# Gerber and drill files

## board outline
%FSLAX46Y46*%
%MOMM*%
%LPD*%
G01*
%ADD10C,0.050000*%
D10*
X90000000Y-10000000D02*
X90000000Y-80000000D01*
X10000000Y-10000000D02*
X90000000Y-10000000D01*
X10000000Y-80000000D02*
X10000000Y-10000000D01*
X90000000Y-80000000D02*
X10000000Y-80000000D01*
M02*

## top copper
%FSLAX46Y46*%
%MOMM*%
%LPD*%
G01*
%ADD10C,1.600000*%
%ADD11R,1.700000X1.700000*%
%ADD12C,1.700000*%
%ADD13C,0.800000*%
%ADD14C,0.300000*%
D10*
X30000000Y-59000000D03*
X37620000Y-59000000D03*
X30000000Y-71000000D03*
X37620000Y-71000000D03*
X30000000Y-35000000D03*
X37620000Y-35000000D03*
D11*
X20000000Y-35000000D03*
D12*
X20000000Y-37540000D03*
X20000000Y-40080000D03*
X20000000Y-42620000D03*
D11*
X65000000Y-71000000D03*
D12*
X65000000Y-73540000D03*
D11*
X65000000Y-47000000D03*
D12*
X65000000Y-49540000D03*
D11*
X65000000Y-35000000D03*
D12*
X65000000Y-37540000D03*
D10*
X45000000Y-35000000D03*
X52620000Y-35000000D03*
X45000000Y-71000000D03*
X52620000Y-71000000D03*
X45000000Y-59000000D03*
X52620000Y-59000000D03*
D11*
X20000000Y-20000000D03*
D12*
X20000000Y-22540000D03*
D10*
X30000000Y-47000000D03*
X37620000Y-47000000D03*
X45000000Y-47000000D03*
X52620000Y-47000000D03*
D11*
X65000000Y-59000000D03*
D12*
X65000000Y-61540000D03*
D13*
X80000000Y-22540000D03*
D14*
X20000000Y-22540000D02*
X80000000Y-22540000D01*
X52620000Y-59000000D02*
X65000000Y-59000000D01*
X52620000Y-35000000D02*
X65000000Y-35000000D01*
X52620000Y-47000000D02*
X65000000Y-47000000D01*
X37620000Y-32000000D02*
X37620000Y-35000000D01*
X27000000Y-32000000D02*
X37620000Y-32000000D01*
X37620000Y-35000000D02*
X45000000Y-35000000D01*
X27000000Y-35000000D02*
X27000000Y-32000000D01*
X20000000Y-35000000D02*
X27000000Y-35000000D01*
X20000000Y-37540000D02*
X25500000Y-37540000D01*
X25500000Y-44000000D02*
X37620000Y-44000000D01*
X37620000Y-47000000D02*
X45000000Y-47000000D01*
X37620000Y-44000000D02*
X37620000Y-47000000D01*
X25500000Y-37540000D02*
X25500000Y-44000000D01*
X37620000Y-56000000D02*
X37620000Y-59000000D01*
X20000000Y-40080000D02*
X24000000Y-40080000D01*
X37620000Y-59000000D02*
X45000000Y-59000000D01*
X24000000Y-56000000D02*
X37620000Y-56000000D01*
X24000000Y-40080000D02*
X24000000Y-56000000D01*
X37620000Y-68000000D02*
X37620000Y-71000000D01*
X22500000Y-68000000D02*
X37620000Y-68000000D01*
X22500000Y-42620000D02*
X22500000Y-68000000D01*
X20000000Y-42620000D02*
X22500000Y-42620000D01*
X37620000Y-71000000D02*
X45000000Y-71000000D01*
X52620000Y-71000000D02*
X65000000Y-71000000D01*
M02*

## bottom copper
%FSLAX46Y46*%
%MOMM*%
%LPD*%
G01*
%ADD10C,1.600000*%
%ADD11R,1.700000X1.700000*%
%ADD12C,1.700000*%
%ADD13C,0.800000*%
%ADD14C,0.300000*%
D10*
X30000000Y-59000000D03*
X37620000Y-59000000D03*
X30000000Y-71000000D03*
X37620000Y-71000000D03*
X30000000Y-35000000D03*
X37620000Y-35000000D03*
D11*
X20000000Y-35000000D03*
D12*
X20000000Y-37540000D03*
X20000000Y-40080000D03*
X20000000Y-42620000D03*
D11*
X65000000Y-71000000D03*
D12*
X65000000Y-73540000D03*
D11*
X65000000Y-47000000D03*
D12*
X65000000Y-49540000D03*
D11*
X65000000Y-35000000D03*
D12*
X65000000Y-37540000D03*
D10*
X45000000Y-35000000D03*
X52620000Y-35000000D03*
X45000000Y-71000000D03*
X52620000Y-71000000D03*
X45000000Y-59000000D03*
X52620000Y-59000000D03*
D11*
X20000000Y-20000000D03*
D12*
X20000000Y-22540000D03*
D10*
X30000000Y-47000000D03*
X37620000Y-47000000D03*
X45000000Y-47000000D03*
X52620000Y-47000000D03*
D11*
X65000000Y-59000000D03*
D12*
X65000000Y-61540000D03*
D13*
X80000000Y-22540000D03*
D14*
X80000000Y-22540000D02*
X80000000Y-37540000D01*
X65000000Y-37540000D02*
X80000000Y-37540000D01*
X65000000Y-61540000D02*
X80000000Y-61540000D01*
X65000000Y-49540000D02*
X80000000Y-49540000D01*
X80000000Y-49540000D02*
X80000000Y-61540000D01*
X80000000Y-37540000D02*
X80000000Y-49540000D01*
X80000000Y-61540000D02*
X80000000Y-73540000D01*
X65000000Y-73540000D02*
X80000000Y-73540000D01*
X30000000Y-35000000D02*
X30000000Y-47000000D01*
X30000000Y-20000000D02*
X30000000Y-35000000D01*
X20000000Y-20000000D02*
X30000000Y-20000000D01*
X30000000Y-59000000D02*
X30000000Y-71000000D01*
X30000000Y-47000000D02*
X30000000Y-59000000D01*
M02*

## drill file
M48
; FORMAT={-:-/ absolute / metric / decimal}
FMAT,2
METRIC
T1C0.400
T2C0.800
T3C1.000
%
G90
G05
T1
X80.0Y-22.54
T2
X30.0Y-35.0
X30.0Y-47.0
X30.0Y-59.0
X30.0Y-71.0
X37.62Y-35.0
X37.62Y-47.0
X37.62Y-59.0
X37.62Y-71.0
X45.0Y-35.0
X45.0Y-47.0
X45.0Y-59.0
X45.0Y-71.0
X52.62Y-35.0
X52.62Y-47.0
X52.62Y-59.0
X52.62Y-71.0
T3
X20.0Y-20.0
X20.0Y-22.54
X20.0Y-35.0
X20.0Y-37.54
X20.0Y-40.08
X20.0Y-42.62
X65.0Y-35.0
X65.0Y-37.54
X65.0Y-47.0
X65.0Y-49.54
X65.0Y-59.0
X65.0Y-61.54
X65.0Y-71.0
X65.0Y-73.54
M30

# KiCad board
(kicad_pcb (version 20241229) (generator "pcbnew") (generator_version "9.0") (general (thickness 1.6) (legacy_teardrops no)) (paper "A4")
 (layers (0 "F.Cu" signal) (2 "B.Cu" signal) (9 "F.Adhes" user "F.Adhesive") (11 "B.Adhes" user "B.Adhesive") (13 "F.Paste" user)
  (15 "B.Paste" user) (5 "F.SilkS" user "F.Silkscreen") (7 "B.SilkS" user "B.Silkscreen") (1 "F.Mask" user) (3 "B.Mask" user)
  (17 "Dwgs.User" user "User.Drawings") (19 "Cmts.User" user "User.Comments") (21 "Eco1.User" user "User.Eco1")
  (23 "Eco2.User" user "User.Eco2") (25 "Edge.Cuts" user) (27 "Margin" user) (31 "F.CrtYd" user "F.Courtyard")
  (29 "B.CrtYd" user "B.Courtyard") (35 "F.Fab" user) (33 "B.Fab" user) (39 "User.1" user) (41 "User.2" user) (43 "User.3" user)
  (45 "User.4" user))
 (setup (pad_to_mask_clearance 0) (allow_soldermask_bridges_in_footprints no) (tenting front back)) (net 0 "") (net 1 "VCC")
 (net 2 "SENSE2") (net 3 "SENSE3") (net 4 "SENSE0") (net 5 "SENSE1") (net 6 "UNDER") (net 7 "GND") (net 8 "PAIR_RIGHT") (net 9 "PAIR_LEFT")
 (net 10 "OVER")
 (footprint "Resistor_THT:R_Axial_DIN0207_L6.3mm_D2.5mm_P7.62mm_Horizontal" (layer "F.Cu") (at 30 59)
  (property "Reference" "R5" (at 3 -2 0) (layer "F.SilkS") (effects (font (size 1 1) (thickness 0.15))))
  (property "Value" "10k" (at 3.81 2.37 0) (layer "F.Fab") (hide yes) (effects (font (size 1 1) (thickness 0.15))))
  (pad "1" thru_hole circle (at 0 0) (size 1.6 1.6) (drill 0.8) (layers "*.Cu" "*.Mask") (remove_unused_layers no) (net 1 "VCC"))
  (pad "2" thru_hole circle (at 7.62 0) (size 1.6 1.6) (drill 0.8) (layers "*.Cu" "*.Mask") (remove_unused_layers no) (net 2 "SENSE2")))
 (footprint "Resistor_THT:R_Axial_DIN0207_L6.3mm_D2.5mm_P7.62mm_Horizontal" (layer "F.Cu") (at 30 71)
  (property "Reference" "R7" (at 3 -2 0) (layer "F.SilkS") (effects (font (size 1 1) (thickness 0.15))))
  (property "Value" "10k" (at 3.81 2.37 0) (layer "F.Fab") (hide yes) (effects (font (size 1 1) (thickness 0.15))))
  (pad "1" thru_hole circle (at 0 0) (size 1.6 1.6) (drill 0.8) (layers "*.Cu" "*.Mask") (remove_unused_layers no) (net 1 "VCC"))
  (pad "2" thru_hole circle (at 7.62 0) (size 1.6 1.6) (drill 0.8) (layers "*.Cu" "*.Mask") (remove_unused_layers no) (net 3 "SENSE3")))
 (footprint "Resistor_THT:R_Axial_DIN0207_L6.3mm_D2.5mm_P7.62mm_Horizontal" (layer "F.Cu") (at 30 35)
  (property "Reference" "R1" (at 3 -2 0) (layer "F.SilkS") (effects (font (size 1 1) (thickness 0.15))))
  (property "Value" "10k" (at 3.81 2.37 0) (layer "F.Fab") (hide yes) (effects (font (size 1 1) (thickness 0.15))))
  (pad "1" thru_hole circle (at 0 0) (size 1.6 1.6) (drill 0.8) (layers "*.Cu" "*.Mask") (remove_unused_layers no) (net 1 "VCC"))
  (pad "2" thru_hole circle (at 7.62 0) (size 1.6 1.6) (drill 0.8) (layers "*.Cu" "*.Mask") (remove_unused_layers no) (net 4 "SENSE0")))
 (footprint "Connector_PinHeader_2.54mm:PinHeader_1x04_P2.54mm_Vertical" (layer "F.Cu") (at 20 35)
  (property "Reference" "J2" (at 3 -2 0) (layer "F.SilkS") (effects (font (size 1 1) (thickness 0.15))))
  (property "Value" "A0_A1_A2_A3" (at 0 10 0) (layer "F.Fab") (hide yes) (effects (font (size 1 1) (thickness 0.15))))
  (pad "1" thru_hole rect (at 0 0) (size 1.7 1.7) (drill 1) (layers "*.Cu" "*.Mask") (remove_unused_layers no) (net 4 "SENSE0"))
  (pad "2" thru_hole circle (at 0 2.54) (size 1.7 1.7) (drill 1) (layers "*.Cu" "*.Mask") (remove_unused_layers no) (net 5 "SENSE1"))
  (pad "3" thru_hole circle (at 0 5.08) (size 1.7 1.7) (drill 1) (layers "*.Cu" "*.Mask") (remove_unused_layers no) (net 2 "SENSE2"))
  (pad "4" thru_hole circle (at 0 7.62) (size 1.7 1.7) (drill 1) (layers "*.Cu" "*.Mask") (remove_unused_layers no) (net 3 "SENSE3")))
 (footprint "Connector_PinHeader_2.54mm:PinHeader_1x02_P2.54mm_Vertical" (layer "F.Cu") (at 65 71)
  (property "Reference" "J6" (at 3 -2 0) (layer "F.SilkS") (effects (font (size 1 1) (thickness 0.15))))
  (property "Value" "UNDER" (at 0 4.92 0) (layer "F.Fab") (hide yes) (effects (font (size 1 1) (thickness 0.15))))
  (pad "1" thru_hole rect (at 0 0) (size 1.7 1.7) (drill 1) (layers "*.Cu" "*.Mask") (remove_unused_layers no) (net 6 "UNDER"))
  (pad "2" thru_hole circle (at 0 2.54) (size 1.7 1.7) (drill 1) (layers "*.Cu" "*.Mask") (remove_unused_layers no) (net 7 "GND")))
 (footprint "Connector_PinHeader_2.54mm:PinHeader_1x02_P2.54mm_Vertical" (layer "F.Cu") (at 65 47)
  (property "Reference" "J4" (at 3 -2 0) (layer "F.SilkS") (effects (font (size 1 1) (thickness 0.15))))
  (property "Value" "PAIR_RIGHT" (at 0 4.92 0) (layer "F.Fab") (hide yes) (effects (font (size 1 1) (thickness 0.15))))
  (pad "1" thru_hole rect (at 0 0) (size 1.7 1.7) (drill 1) (layers "*.Cu" "*.Mask") (remove_unused_layers no) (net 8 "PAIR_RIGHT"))
  (pad "2" thru_hole circle (at 0 2.54) (size 1.7 1.7) (drill 1) (layers "*.Cu" "*.Mask") (remove_unused_layers no) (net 7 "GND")))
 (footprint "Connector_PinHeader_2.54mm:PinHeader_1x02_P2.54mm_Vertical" (layer "F.Cu") (at 65 35)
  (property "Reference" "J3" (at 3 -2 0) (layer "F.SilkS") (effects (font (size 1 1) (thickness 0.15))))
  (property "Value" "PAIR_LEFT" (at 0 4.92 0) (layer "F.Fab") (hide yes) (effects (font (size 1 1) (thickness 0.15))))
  (pad "1" thru_hole rect (at 0 0) (size 1.7 1.7) (drill 1) (layers "*.Cu" "*.Mask") (remove_unused_layers no) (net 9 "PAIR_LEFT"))
  (pad "2" thru_hole circle (at 0 2.54) (size 1.7 1.7) (drill 1) (layers "*.Cu" "*.Mask") (remove_unused_layers no) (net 7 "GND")))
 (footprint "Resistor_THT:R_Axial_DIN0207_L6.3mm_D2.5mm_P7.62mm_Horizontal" (layer "F.Cu") (at 45 35)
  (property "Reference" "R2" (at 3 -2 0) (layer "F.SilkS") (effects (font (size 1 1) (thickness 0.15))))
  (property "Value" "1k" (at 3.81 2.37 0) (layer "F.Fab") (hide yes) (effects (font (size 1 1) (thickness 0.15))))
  (pad "1" thru_hole circle (at 0 0) (size 1.6 1.6) (drill 0.8) (layers "*.Cu" "*.Mask") (remove_unused_layers no) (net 4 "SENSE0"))
  (pad "2" thru_hole circle (at 7.62 0) (size 1.6 1.6) (drill 0.8) (layers "*.Cu" "*.Mask") (remove_unused_layers no) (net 9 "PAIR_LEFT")))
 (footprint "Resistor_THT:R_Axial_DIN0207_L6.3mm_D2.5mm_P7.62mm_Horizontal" (layer "F.Cu") (at 45 71)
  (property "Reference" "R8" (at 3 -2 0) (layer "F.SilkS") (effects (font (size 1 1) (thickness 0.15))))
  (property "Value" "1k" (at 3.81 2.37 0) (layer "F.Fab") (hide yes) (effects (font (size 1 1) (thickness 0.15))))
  (pad "1" thru_hole circle (at 0 0) (size 1.6 1.6) (drill 0.8) (layers "*.Cu" "*.Mask") (remove_unused_layers no) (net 3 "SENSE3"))
  (pad "2" thru_hole circle (at 7.62 0) (size 1.6 1.6) (drill 0.8) (layers "*.Cu" "*.Mask") (remove_unused_layers no) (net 6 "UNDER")))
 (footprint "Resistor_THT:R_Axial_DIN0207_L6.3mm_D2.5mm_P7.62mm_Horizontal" (layer "F.Cu") (at 45 59)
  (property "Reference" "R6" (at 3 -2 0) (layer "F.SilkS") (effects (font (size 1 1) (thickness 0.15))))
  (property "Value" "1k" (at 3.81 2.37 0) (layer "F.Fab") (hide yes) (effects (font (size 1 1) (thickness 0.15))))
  (pad "1" thru_hole circle (at 0 0) (size 1.6 1.6) (drill 0.8) (layers "*.Cu" "*.Mask") (remove_unused_layers no) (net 2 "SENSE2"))
  (pad "2" thru_hole circle (at 7.62 0) (size 1.6 1.6) (drill 0.8) (layers "*.Cu" "*.Mask") (remove_unused_layers no) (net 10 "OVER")))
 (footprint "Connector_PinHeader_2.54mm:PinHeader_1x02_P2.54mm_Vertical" (layer "F.Cu") (at 20 20)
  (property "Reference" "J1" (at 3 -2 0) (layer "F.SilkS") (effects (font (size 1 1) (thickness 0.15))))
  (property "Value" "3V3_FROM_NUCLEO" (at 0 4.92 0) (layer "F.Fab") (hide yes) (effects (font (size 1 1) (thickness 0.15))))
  (pad "1" thru_hole rect (at 0 0) (size 1.7 1.7) (drill 1) (layers "*.Cu" "*.Mask") (remove_unused_layers no) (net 1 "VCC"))
  (pad "2" thru_hole circle (at 0 2.54) (size 1.7 1.7) (drill 1) (layers "*.Cu" "*.Mask") (remove_unused_layers no) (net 7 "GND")))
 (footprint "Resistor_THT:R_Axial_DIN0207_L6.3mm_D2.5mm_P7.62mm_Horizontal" (layer "F.Cu") (at 30 47)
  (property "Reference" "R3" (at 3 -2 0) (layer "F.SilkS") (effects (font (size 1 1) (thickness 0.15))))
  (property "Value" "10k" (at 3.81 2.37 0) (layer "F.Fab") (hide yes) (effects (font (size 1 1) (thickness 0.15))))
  (pad "1" thru_hole circle (at 0 0) (size 1.6 1.6) (drill 0.8) (layers "*.Cu" "*.Mask") (remove_unused_layers no) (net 1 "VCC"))
  (pad "2" thru_hole circle (at 7.62 0) (size 1.6 1.6) (drill 0.8) (layers "*.Cu" "*.Mask") (remove_unused_layers no) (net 5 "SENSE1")))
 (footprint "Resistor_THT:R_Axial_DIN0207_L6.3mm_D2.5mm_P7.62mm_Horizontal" (layer "F.Cu") (at 45 47)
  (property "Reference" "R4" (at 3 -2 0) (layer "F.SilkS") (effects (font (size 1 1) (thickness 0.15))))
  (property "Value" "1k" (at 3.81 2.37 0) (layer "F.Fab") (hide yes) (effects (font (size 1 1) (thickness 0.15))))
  (pad "1" thru_hole circle (at 0 0) (size 1.6 1.6) (drill 0.8) (layers "*.Cu" "*.Mask") (remove_unused_layers no) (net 5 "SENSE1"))
  (pad "2" thru_hole circle (at 7.62 0) (size 1.6 1.6) (drill 0.8) (layers "*.Cu" "*.Mask") (remove_unused_layers no) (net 8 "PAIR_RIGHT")))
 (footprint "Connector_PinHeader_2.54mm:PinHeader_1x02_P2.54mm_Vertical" (layer "F.Cu") (at 65 59)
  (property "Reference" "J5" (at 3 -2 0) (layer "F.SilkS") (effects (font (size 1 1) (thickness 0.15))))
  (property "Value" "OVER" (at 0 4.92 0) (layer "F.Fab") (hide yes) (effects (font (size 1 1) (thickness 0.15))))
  (pad "1" thru_hole rect (at 0 0) (size 1.7 1.7) (drill 1) (layers "*.Cu" "*.Mask") (remove_unused_layers no) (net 10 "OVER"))
  (pad "2" thru_hole circle (at 0 2.54) (size 1.7 1.7) (drill 1) (layers "*.Cu" "*.Mask") (remove_unused_layers no) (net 7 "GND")))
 (gr_line (start 90 10) (end 90 80) (stroke (width 0.05) (type default)) (layer "Edge.Cuts"))
 (gr_line (start 10 10) (end 90 10) (stroke (width 0.05) (type default)) (layer "Edge.Cuts"))
 (gr_line (start 10 80) (end 10 10) (stroke (width 0.05) (type default)) (layer "Edge.Cuts"))
 (gr_line (start 90 80) (end 10 80) (stroke (width 0.05) (type default)) (layer "Edge.Cuts"))
 (segment (start 20 22.54) (end 80 22.54) (width 0.3) (layer "F.Cu") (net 7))
 (via (at 80 22.54) (size 0.8) (drill 0.4) (layers "F.Cu" "B.Cu") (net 7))
 (segment (start 80 22.54) (end 80 37.54) (width 0.3) (layer "B.Cu") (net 7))
 (segment (start 65 37.54) (end 80 37.54) (width 0.3) (layer "B.Cu") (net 7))
 (segment (start 65 61.54) (end 80 61.54) (width 0.3) (layer "B.Cu") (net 7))
 (segment (start 65 49.54) (end 80 49.54) (width 0.3) (layer "B.Cu") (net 7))
 (segment (start 80 49.54) (end 80 61.54) (width 0.3) (layer "B.Cu") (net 7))
 (segment (start 80 37.54) (end 80 49.54) (width 0.3) (layer "B.Cu") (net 7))
 (segment (start 80 61.54) (end 80 73.54) (width 0.3) (layer "B.Cu") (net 7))
 (segment (start 65 73.54) (end 80 73.54) (width 0.3) (layer "B.Cu") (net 7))
 (segment (start 52.62 59) (end 65 59) (width 0.3) (layer "F.Cu") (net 10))
 (segment (start 52.62 35) (end 65 35) (width 0.3) (layer "F.Cu") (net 9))
 (segment (start 52.62 47) (end 65 47) (width 0.3) (layer "F.Cu") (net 8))
 (segment (start 37.62 32) (end 37.62 35) (width 0.3) (layer "F.Cu") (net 4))
 (segment (start 27 32) (end 37.62 32) (width 0.3) (layer "F.Cu") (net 4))
 (segment (start 37.62 35) (end 45 35) (width 0.3) (layer "F.Cu") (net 4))
 (segment (start 27 35) (end 27 32) (width 0.3) (layer "F.Cu") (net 4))
 (segment (start 20 35) (end 27 35) (width 0.3) (layer "F.Cu") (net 4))
 (segment (start 20 37.54) (end 25.5 37.54) (width 0.3) (layer "F.Cu") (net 5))
 (segment (start 25.5 44) (end 37.62 44) (width 0.3) (layer "F.Cu") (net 5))
 (segment (start 37.62 47) (end 45 47) (width 0.3) (layer "F.Cu") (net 5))
 (segment (start 37.62 44) (end 37.62 47) (width 0.3) (layer "F.Cu") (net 5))
 (segment (start 25.5 37.54) (end 25.5 44) (width 0.3) (layer "F.Cu") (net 5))
 (segment (start 37.62 56) (end 37.62 59) (width 0.3) (layer "F.Cu") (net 2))
 (segment (start 20 40.08) (end 24 40.08) (width 0.3) (layer "F.Cu") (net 2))
 (segment (start 37.62 59) (end 45 59) (width 0.3) (layer "F.Cu") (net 2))
 (segment (start 24 56) (end 37.62 56) (width 0.3) (layer "F.Cu") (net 2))
 (segment (start 24 40.08) (end 24 56) (width 0.3) (layer "F.Cu") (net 2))
 (segment (start 37.62 68) (end 37.62 71) (width 0.3) (layer "F.Cu") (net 3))
 (segment (start 22.5 68) (end 37.62 68) (width 0.3) (layer "F.Cu") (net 3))
 (segment (start 22.5 42.62) (end 22.5 68) (width 0.3) (layer "F.Cu") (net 3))
 (segment (start 20 42.62) (end 22.5 42.62) (width 0.3) (layer "F.Cu") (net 3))
 (segment (start 37.62 71) (end 45 71) (width 0.3) (layer "F.Cu") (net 3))
 (segment (start 52.62 71) (end 65 71) (width 0.3) (layer "F.Cu") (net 6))
 (segment (start 30 35) (end 30 47) (width 0.3) (layer "B.Cu") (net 1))
 (segment (start 30 20) (end 30 35) (width 0.3) (layer "B.Cu") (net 1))
 (segment (start 20 20) (end 30 20) (width 0.3) (layer "B.Cu") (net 1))
 (segment (start 30 59) (end 30 71) (width 0.3) (layer "B.Cu") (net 1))
 (segment (start 30 47) (end 30 59) (width 0.3) (layer "B.Cu") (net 1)))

